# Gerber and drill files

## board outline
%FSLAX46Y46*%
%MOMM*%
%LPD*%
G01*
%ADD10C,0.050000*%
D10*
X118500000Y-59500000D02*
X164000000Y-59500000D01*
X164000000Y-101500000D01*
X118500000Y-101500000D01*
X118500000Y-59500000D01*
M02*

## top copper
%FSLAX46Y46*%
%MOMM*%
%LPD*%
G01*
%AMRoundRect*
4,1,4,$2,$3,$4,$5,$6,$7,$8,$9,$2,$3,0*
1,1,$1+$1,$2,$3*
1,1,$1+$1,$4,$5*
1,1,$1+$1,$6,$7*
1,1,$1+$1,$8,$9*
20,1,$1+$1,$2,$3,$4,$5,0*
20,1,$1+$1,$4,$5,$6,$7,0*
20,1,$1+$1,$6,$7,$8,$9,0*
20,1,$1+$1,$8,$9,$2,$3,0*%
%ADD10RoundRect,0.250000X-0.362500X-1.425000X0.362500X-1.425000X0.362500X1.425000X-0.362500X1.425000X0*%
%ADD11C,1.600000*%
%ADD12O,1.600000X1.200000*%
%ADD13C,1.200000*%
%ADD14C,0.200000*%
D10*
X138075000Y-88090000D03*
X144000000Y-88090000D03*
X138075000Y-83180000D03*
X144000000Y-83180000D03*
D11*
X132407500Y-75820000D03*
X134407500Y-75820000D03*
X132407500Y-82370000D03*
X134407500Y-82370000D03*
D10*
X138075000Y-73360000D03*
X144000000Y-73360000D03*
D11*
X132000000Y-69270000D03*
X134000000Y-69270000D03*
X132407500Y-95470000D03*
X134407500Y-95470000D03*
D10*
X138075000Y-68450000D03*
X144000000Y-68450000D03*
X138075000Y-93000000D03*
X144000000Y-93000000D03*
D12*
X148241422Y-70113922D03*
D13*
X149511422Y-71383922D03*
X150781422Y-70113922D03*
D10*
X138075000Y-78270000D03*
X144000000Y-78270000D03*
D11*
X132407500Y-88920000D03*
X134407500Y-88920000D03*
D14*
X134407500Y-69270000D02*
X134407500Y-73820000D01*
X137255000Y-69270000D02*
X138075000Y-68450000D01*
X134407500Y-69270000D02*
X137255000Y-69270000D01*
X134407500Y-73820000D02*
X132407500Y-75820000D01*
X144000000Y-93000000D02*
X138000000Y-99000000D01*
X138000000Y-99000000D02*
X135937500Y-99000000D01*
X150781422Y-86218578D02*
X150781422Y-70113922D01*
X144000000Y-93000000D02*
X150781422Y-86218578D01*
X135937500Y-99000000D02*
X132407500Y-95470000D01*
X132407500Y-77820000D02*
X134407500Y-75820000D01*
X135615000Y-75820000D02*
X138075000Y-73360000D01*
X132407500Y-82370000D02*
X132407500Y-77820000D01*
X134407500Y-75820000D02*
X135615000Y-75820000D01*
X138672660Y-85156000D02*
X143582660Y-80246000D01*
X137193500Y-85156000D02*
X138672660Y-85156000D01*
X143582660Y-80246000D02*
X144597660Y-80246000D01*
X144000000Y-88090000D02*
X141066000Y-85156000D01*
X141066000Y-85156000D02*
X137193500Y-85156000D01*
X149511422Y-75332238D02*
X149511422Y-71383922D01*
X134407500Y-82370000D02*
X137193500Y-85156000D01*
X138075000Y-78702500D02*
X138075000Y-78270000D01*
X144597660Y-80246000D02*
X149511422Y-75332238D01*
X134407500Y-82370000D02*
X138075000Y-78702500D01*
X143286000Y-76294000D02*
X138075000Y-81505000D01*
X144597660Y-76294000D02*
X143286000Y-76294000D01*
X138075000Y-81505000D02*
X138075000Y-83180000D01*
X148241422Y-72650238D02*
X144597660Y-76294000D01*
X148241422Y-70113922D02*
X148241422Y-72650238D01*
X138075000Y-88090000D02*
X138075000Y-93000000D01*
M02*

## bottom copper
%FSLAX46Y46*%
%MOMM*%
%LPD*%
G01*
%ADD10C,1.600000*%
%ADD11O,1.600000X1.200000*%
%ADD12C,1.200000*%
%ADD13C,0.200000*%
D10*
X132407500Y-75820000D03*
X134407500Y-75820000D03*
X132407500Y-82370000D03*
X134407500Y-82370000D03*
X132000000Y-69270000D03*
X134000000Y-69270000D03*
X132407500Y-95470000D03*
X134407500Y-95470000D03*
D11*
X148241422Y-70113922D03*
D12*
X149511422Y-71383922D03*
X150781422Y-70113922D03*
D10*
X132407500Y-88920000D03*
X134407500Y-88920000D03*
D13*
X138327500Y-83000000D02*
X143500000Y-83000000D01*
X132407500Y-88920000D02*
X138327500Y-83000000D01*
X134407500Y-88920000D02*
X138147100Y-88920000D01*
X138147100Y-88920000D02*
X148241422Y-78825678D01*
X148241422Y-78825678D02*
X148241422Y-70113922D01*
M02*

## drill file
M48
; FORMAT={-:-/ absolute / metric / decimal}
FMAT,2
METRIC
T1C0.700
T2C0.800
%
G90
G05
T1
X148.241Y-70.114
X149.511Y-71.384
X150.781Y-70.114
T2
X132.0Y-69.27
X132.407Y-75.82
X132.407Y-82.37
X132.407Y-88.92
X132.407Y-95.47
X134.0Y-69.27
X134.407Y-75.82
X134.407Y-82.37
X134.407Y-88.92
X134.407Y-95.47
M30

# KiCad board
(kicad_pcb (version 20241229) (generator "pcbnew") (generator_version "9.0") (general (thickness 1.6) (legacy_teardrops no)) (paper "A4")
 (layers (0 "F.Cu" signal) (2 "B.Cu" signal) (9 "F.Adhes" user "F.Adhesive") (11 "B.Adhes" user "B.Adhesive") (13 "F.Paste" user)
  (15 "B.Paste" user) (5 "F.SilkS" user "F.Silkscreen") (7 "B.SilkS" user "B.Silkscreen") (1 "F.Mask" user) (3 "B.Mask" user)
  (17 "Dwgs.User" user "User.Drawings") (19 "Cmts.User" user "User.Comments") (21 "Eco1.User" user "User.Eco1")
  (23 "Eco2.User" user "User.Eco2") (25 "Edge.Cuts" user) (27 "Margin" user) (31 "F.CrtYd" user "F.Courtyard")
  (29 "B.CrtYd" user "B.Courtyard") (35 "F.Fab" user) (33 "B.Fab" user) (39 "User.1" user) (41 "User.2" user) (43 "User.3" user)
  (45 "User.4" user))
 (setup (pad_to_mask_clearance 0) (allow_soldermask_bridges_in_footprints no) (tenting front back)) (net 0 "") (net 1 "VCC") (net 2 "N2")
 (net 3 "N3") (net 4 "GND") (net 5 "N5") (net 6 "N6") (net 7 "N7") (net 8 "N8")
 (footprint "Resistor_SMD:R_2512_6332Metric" (layer "F.Cu") (at 141.0375 88.09)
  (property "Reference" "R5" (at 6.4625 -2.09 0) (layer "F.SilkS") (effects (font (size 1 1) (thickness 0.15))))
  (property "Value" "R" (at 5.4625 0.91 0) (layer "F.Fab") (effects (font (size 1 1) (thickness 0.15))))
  (pad "1" smd roundrect (at -2.9625 0) (size 1.225 3.35) (layers "F.Cu" "F.Mask" "F.Paste") (roundrect_rratio 0.204082) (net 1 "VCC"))
  (pad "2" smd roundrect (at 2.9625 0) (size 1.225 3.35) (layers "F.Cu" "F.Mask" "F.Paste") (roundrect_rratio 0.204082) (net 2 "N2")))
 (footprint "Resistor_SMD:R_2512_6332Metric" (layer "F.Cu") (at 141.0375 83.18)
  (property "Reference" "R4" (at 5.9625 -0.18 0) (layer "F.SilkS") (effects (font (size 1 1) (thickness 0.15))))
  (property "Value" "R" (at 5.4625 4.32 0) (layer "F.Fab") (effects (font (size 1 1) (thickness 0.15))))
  (pad "1" smd roundrect (at -2.9625 0) (size 1.225 3.35) (layers "F.Cu" "F.Mask" "F.Paste") (roundrect_rratio 0.204082) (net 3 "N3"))
  (pad "2" smd roundrect (at 2.9625 0) (size 1.225 3.35) (layers "F.Cu" "F.Mask" "F.Paste") (roundrect_rratio 0.204082) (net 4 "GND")))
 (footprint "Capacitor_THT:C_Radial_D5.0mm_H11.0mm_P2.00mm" (layer "F.Cu") (at 132.4075 75.82)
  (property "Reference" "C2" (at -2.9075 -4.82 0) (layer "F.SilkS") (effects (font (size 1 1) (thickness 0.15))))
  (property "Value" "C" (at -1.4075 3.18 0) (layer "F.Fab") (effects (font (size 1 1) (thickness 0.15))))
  (pad "1" thru_hole circle (at 0 0) (size 1.6 1.6) (drill 0.8) (layers "*.Cu" "*.Mask") (remove_unused_layers no) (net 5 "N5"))
  (pad "2" thru_hole circle (at 2 0) (size 1.6 1.6) (drill 0.8) (layers "*.Cu" "*.Mask") (remove_unused_layers no) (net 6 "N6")))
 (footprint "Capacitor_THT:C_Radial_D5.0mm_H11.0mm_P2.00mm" (layer "F.Cu") (at 132.4075 82.37)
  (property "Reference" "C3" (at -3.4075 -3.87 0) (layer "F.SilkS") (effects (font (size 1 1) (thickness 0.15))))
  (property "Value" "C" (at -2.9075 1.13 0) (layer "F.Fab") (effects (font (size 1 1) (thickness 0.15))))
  (pad "1" thru_hole circle (at 0 0) (size 1.6 1.6) (drill 0.8) (layers "*.Cu" "*.Mask") (remove_unused_layers no) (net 6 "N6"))
  (pad "2" thru_hole circle (at 2 0) (size 1.6 1.6) (drill 0.8) (layers "*.Cu" "*.Mask") (remove_unused_layers no) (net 2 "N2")))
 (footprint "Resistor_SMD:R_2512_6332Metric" (layer "F.Cu") (at 141.0375 73.36)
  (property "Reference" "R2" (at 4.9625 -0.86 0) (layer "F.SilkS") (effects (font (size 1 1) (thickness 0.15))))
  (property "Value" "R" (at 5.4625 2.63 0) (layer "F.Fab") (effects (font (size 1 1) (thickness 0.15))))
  (pad "1" smd roundrect (at -2.9625 0) (size 1.225 3.35) (layers "F.Cu" "F.Mask" "F.Paste") (roundrect_rratio 0.204082) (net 6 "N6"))
  (pad "2" smd roundrect (at 2.9625 0) (size 1.225 3.35) (layers "F.Cu" "F.Mask" "F.Paste") (roundrect_rratio 0.204082) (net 4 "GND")))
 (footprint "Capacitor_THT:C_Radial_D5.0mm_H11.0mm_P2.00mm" (layer "F.Cu") (at 132 69.27)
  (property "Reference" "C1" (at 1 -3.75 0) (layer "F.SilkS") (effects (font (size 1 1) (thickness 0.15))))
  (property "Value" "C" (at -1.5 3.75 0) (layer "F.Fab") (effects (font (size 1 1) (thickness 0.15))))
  (pad "1" thru_hole circle (at 0 0) (size 1.6 1.6) (drill 0.8) (layers "*.Cu" "*.Mask") (remove_unused_layers no) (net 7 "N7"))
  (pad "2" thru_hole circle (at 2 0) (size 1.6 1.6) (drill 0.8) (layers "*.Cu" "*.Mask") (remove_unused_layers no) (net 5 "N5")))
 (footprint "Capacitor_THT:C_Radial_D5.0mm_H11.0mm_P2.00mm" (layer "F.Cu") (at 132.4075 95.47)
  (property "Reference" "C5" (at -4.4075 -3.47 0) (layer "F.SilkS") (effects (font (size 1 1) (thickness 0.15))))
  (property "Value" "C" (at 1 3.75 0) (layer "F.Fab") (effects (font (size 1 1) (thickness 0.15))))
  (pad "1" thru_hole circle (at 0 0) (size 1.6 1.6) (drill 0.8) (layers "*.Cu" "*.Mask") (remove_unused_layers no) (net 7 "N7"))
  (pad "2" thru_hole circle (at 2 0) (size 1.6 1.6) (drill 0.8) (layers "*.Cu" "*.Mask") (remove_unused_layers no) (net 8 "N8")))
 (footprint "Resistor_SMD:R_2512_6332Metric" (layer "F.Cu") (at 141.0375 68.45)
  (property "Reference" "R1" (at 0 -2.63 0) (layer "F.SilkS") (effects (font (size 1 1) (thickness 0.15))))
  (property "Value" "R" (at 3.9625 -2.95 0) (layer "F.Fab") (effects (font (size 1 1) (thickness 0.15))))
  (pad "1" smd roundrect (at -2.9625 0) (size 1.225 3.35) (layers "F.Cu" "F.Mask" "F.Paste") (roundrect_rratio 0.204082) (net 5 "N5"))
  (pad "2" smd roundrect (at 2.9625 0) (size 1.225 3.35) (layers "F.Cu" "F.Mask" "F.Paste") (roundrect_rratio 0.204082) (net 4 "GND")))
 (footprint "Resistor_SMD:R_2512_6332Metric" (layer "F.Cu") (at 141.0375 93)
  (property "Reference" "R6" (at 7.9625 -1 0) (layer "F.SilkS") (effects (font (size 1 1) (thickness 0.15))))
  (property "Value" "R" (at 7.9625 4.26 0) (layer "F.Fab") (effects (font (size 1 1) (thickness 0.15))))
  (pad "1" smd roundrect (at -2.9625 0) (size 1.225 3.35) (layers "F.Cu" "F.Mask" "F.Paste") (roundrect_rratio 0.204082) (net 1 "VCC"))
  (pad "2" smd roundrect (at 2.9625 0) (size 1.225 3.35) (layers "F.Cu" "F.Mask" "F.Paste") (roundrect_rratio 0.204082) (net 7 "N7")))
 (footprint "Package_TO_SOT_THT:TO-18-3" (layer "F.Cu") (at 148.241422 70.113922)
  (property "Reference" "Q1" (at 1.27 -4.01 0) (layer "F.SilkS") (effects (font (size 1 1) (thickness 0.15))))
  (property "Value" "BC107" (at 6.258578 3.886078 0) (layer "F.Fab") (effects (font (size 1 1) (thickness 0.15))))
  (pad "1" thru_hole oval (at 0 0) (size 1.6 1.2) (drill 0.7) (layers "*.Cu" "*.Mask") (remove_unused_layers no) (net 3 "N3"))
  (pad "2" thru_hole circle (at 1.27 1.27) (size 1.2 1.2) (drill 0.7) (layers "*.Cu" "*.Mask") (remove_unused_layers no) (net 2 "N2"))
  (pad "3" thru_hole circle (at 2.54 0) (size 1.2 1.2) (drill 0.7) (layers "*.Cu" "*.Mask") (remove_unused_layers no) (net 7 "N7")))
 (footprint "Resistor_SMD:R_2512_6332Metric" (layer "F.Cu") (at 141.0375 78.27)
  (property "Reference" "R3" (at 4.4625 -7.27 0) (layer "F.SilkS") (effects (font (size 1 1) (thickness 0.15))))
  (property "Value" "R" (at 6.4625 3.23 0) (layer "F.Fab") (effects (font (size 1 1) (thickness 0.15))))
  (pad "1" smd roundrect (at -2.9625 0) (size 1.225 3.35) (layers "F.Cu" "F.Mask" "F.Paste") (roundrect_rratio 0.204082) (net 2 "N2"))
  (pad "2" smd roundrect (at 2.9625 0) (size 1.225 3.35) (layers "F.Cu" "F.Mask" "F.Paste") (roundrect_rratio 0.204082) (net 4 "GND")))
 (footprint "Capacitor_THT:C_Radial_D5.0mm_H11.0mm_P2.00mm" (layer "F.Cu") (at 132.4075 88.92)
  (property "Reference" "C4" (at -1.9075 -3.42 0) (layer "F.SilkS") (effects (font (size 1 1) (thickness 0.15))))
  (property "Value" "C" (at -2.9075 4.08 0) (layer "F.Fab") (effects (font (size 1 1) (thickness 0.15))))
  (pad "1" thru_hole circle (at 0 0) (size 1.6 1.6) (drill 0.8) (layers "*.Cu" "*.Mask") (remove_unused_layers no) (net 4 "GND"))
  (pad "2" thru_hole circle (at 2 0) (size 1.6 1.6) (drill 0.8) (layers "*.Cu" "*.Mask") (remove_unused_layers no) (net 3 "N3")))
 (gr_rect (start 118.5 59.5) (end 164 101.5) (stroke (width 0.05) (type default)) (fill no) (layer "Edge.Cuts"))
 (segment (start 134.4075 69.27) (end 134.4075 73.82) (width 0.2) (layer "F.Cu") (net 5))
 (segment (start 137.255 69.27) (end 138.075 68.45) (width 0.2) (layer "F.Cu") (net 5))
 (segment (start 134.4075 69.27) (end 137.255 69.27) (width 0.2) (layer "F.Cu") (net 5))
 (segment (start 134.4075 73.82) (end 132.4075 75.82) (width 0.2) (layer "F.Cu") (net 5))
 (segment (start 144 93) (end 138 99) (width 0.2) (layer "F.Cu") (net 7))
 (segment (start 138 99) (end 135.9375 99) (width 0.2) (layer "F.Cu") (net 7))
 (segment (start 150.781422 86.218578) (end 150.781422 70.113922) (width 0.2) (layer "F.Cu") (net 7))
 (segment (start 144 93) (end 150.781422 86.218578) (width 0.2) (layer "F.Cu") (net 7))
 (segment (start 135.9375 99) (end 132.4075 95.47) (width 0.2) (layer "F.Cu") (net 7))
 (segment (start 132.4075 77.82) (end 134.4075 75.82) (width 0.2) (layer "F.Cu") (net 6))
 (segment (start 135.615 75.82) (end 138.075 73.36) (width 0.2) (layer "F.Cu") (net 6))
 (segment (start 132.4075 82.37) (end 132.4075 77.82) (width 0.2) (layer "F.Cu") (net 6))
 (segment (start 134.4075 75.82) (end 135.615 75.82) (width 0.2) (layer "F.Cu") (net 6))
 (segment (start 138.67266 85.156) (end 143.58266 80.246) (width 0.2) (layer "F.Cu") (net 2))
 (segment (start 137.1935 85.156) (end 138.67266 85.156) (width 0.2) (layer "F.Cu") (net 2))
 (segment (start 143.58266 80.246) (end 144.59766 80.246) (width 0.2) (layer "F.Cu") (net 2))
 (segment (start 144 88.09) (end 141.066 85.156) (width 0.2) (layer "F.Cu") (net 2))
 (segment (start 141.066 85.156) (end 137.1935 85.156) (width 0.2) (layer "F.Cu") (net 2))
 (segment (start 149.511422 75.332238) (end 149.511422 71.383922) (width 0.2) (layer "F.Cu") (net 2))
 (segment (start 134.4075 82.37) (end 137.1935 85.156) (width 0.2) (layer "F.Cu") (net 2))
 (segment (start 138.075 78.7025) (end 138.075 78.27) (width 0.2) (layer "F.Cu") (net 2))
 (segment (start 144.59766 80.246) (end 149.511422 75.332238) (width 0.2) (layer "F.Cu") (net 2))
 (segment (start 134.4075 82.37) (end 138.075 78.7025) (width 0.2) (layer "F.Cu") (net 2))
 (segment (start 138.3275 83) (end 143.5 83) (width 0.2) (layer "B.Cu") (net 4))
 (segment (start 132.4075 88.92) (end 138.3275 83) (width 0.2) (layer "B.Cu") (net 4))
 (segment (start 143.286 76.294) (end 138.075 81.505) (width 0.2) (layer "F.Cu") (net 3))
 (segment (start 144.59766 76.294) (end 143.286 76.294) (width 0.2) (layer "F.Cu") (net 3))
 (segment (start 138.075 81.505) (end 138.075 83.18) (width 0.2) (layer "F.Cu") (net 3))
 (segment (start 148.241422 72.650238) (end 144.59766 76.294) (width 0.2) (layer "F.Cu") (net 3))
 (segment (start 148.241422 70.113922) (end 148.241422 72.650238) (width 0.2) (layer "F.Cu") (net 3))
 (segment (start 134.4075 88.92) (end 138.1471 88.92) (width 0.2) (layer "B.Cu") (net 3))
 (segment (start 138.1471 88.92) (end 148.241422 78.825678) (width 0.2) (layer "B.Cu") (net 3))
 (segment (start 148.241422 78.825678) (end 148.241422 70.113922) (width 0.2) (layer "B.Cu") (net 3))
 (segment (start 138.075 88.09) (end 138.075 93) (width 0.2) (layer "F.Cu") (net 1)))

